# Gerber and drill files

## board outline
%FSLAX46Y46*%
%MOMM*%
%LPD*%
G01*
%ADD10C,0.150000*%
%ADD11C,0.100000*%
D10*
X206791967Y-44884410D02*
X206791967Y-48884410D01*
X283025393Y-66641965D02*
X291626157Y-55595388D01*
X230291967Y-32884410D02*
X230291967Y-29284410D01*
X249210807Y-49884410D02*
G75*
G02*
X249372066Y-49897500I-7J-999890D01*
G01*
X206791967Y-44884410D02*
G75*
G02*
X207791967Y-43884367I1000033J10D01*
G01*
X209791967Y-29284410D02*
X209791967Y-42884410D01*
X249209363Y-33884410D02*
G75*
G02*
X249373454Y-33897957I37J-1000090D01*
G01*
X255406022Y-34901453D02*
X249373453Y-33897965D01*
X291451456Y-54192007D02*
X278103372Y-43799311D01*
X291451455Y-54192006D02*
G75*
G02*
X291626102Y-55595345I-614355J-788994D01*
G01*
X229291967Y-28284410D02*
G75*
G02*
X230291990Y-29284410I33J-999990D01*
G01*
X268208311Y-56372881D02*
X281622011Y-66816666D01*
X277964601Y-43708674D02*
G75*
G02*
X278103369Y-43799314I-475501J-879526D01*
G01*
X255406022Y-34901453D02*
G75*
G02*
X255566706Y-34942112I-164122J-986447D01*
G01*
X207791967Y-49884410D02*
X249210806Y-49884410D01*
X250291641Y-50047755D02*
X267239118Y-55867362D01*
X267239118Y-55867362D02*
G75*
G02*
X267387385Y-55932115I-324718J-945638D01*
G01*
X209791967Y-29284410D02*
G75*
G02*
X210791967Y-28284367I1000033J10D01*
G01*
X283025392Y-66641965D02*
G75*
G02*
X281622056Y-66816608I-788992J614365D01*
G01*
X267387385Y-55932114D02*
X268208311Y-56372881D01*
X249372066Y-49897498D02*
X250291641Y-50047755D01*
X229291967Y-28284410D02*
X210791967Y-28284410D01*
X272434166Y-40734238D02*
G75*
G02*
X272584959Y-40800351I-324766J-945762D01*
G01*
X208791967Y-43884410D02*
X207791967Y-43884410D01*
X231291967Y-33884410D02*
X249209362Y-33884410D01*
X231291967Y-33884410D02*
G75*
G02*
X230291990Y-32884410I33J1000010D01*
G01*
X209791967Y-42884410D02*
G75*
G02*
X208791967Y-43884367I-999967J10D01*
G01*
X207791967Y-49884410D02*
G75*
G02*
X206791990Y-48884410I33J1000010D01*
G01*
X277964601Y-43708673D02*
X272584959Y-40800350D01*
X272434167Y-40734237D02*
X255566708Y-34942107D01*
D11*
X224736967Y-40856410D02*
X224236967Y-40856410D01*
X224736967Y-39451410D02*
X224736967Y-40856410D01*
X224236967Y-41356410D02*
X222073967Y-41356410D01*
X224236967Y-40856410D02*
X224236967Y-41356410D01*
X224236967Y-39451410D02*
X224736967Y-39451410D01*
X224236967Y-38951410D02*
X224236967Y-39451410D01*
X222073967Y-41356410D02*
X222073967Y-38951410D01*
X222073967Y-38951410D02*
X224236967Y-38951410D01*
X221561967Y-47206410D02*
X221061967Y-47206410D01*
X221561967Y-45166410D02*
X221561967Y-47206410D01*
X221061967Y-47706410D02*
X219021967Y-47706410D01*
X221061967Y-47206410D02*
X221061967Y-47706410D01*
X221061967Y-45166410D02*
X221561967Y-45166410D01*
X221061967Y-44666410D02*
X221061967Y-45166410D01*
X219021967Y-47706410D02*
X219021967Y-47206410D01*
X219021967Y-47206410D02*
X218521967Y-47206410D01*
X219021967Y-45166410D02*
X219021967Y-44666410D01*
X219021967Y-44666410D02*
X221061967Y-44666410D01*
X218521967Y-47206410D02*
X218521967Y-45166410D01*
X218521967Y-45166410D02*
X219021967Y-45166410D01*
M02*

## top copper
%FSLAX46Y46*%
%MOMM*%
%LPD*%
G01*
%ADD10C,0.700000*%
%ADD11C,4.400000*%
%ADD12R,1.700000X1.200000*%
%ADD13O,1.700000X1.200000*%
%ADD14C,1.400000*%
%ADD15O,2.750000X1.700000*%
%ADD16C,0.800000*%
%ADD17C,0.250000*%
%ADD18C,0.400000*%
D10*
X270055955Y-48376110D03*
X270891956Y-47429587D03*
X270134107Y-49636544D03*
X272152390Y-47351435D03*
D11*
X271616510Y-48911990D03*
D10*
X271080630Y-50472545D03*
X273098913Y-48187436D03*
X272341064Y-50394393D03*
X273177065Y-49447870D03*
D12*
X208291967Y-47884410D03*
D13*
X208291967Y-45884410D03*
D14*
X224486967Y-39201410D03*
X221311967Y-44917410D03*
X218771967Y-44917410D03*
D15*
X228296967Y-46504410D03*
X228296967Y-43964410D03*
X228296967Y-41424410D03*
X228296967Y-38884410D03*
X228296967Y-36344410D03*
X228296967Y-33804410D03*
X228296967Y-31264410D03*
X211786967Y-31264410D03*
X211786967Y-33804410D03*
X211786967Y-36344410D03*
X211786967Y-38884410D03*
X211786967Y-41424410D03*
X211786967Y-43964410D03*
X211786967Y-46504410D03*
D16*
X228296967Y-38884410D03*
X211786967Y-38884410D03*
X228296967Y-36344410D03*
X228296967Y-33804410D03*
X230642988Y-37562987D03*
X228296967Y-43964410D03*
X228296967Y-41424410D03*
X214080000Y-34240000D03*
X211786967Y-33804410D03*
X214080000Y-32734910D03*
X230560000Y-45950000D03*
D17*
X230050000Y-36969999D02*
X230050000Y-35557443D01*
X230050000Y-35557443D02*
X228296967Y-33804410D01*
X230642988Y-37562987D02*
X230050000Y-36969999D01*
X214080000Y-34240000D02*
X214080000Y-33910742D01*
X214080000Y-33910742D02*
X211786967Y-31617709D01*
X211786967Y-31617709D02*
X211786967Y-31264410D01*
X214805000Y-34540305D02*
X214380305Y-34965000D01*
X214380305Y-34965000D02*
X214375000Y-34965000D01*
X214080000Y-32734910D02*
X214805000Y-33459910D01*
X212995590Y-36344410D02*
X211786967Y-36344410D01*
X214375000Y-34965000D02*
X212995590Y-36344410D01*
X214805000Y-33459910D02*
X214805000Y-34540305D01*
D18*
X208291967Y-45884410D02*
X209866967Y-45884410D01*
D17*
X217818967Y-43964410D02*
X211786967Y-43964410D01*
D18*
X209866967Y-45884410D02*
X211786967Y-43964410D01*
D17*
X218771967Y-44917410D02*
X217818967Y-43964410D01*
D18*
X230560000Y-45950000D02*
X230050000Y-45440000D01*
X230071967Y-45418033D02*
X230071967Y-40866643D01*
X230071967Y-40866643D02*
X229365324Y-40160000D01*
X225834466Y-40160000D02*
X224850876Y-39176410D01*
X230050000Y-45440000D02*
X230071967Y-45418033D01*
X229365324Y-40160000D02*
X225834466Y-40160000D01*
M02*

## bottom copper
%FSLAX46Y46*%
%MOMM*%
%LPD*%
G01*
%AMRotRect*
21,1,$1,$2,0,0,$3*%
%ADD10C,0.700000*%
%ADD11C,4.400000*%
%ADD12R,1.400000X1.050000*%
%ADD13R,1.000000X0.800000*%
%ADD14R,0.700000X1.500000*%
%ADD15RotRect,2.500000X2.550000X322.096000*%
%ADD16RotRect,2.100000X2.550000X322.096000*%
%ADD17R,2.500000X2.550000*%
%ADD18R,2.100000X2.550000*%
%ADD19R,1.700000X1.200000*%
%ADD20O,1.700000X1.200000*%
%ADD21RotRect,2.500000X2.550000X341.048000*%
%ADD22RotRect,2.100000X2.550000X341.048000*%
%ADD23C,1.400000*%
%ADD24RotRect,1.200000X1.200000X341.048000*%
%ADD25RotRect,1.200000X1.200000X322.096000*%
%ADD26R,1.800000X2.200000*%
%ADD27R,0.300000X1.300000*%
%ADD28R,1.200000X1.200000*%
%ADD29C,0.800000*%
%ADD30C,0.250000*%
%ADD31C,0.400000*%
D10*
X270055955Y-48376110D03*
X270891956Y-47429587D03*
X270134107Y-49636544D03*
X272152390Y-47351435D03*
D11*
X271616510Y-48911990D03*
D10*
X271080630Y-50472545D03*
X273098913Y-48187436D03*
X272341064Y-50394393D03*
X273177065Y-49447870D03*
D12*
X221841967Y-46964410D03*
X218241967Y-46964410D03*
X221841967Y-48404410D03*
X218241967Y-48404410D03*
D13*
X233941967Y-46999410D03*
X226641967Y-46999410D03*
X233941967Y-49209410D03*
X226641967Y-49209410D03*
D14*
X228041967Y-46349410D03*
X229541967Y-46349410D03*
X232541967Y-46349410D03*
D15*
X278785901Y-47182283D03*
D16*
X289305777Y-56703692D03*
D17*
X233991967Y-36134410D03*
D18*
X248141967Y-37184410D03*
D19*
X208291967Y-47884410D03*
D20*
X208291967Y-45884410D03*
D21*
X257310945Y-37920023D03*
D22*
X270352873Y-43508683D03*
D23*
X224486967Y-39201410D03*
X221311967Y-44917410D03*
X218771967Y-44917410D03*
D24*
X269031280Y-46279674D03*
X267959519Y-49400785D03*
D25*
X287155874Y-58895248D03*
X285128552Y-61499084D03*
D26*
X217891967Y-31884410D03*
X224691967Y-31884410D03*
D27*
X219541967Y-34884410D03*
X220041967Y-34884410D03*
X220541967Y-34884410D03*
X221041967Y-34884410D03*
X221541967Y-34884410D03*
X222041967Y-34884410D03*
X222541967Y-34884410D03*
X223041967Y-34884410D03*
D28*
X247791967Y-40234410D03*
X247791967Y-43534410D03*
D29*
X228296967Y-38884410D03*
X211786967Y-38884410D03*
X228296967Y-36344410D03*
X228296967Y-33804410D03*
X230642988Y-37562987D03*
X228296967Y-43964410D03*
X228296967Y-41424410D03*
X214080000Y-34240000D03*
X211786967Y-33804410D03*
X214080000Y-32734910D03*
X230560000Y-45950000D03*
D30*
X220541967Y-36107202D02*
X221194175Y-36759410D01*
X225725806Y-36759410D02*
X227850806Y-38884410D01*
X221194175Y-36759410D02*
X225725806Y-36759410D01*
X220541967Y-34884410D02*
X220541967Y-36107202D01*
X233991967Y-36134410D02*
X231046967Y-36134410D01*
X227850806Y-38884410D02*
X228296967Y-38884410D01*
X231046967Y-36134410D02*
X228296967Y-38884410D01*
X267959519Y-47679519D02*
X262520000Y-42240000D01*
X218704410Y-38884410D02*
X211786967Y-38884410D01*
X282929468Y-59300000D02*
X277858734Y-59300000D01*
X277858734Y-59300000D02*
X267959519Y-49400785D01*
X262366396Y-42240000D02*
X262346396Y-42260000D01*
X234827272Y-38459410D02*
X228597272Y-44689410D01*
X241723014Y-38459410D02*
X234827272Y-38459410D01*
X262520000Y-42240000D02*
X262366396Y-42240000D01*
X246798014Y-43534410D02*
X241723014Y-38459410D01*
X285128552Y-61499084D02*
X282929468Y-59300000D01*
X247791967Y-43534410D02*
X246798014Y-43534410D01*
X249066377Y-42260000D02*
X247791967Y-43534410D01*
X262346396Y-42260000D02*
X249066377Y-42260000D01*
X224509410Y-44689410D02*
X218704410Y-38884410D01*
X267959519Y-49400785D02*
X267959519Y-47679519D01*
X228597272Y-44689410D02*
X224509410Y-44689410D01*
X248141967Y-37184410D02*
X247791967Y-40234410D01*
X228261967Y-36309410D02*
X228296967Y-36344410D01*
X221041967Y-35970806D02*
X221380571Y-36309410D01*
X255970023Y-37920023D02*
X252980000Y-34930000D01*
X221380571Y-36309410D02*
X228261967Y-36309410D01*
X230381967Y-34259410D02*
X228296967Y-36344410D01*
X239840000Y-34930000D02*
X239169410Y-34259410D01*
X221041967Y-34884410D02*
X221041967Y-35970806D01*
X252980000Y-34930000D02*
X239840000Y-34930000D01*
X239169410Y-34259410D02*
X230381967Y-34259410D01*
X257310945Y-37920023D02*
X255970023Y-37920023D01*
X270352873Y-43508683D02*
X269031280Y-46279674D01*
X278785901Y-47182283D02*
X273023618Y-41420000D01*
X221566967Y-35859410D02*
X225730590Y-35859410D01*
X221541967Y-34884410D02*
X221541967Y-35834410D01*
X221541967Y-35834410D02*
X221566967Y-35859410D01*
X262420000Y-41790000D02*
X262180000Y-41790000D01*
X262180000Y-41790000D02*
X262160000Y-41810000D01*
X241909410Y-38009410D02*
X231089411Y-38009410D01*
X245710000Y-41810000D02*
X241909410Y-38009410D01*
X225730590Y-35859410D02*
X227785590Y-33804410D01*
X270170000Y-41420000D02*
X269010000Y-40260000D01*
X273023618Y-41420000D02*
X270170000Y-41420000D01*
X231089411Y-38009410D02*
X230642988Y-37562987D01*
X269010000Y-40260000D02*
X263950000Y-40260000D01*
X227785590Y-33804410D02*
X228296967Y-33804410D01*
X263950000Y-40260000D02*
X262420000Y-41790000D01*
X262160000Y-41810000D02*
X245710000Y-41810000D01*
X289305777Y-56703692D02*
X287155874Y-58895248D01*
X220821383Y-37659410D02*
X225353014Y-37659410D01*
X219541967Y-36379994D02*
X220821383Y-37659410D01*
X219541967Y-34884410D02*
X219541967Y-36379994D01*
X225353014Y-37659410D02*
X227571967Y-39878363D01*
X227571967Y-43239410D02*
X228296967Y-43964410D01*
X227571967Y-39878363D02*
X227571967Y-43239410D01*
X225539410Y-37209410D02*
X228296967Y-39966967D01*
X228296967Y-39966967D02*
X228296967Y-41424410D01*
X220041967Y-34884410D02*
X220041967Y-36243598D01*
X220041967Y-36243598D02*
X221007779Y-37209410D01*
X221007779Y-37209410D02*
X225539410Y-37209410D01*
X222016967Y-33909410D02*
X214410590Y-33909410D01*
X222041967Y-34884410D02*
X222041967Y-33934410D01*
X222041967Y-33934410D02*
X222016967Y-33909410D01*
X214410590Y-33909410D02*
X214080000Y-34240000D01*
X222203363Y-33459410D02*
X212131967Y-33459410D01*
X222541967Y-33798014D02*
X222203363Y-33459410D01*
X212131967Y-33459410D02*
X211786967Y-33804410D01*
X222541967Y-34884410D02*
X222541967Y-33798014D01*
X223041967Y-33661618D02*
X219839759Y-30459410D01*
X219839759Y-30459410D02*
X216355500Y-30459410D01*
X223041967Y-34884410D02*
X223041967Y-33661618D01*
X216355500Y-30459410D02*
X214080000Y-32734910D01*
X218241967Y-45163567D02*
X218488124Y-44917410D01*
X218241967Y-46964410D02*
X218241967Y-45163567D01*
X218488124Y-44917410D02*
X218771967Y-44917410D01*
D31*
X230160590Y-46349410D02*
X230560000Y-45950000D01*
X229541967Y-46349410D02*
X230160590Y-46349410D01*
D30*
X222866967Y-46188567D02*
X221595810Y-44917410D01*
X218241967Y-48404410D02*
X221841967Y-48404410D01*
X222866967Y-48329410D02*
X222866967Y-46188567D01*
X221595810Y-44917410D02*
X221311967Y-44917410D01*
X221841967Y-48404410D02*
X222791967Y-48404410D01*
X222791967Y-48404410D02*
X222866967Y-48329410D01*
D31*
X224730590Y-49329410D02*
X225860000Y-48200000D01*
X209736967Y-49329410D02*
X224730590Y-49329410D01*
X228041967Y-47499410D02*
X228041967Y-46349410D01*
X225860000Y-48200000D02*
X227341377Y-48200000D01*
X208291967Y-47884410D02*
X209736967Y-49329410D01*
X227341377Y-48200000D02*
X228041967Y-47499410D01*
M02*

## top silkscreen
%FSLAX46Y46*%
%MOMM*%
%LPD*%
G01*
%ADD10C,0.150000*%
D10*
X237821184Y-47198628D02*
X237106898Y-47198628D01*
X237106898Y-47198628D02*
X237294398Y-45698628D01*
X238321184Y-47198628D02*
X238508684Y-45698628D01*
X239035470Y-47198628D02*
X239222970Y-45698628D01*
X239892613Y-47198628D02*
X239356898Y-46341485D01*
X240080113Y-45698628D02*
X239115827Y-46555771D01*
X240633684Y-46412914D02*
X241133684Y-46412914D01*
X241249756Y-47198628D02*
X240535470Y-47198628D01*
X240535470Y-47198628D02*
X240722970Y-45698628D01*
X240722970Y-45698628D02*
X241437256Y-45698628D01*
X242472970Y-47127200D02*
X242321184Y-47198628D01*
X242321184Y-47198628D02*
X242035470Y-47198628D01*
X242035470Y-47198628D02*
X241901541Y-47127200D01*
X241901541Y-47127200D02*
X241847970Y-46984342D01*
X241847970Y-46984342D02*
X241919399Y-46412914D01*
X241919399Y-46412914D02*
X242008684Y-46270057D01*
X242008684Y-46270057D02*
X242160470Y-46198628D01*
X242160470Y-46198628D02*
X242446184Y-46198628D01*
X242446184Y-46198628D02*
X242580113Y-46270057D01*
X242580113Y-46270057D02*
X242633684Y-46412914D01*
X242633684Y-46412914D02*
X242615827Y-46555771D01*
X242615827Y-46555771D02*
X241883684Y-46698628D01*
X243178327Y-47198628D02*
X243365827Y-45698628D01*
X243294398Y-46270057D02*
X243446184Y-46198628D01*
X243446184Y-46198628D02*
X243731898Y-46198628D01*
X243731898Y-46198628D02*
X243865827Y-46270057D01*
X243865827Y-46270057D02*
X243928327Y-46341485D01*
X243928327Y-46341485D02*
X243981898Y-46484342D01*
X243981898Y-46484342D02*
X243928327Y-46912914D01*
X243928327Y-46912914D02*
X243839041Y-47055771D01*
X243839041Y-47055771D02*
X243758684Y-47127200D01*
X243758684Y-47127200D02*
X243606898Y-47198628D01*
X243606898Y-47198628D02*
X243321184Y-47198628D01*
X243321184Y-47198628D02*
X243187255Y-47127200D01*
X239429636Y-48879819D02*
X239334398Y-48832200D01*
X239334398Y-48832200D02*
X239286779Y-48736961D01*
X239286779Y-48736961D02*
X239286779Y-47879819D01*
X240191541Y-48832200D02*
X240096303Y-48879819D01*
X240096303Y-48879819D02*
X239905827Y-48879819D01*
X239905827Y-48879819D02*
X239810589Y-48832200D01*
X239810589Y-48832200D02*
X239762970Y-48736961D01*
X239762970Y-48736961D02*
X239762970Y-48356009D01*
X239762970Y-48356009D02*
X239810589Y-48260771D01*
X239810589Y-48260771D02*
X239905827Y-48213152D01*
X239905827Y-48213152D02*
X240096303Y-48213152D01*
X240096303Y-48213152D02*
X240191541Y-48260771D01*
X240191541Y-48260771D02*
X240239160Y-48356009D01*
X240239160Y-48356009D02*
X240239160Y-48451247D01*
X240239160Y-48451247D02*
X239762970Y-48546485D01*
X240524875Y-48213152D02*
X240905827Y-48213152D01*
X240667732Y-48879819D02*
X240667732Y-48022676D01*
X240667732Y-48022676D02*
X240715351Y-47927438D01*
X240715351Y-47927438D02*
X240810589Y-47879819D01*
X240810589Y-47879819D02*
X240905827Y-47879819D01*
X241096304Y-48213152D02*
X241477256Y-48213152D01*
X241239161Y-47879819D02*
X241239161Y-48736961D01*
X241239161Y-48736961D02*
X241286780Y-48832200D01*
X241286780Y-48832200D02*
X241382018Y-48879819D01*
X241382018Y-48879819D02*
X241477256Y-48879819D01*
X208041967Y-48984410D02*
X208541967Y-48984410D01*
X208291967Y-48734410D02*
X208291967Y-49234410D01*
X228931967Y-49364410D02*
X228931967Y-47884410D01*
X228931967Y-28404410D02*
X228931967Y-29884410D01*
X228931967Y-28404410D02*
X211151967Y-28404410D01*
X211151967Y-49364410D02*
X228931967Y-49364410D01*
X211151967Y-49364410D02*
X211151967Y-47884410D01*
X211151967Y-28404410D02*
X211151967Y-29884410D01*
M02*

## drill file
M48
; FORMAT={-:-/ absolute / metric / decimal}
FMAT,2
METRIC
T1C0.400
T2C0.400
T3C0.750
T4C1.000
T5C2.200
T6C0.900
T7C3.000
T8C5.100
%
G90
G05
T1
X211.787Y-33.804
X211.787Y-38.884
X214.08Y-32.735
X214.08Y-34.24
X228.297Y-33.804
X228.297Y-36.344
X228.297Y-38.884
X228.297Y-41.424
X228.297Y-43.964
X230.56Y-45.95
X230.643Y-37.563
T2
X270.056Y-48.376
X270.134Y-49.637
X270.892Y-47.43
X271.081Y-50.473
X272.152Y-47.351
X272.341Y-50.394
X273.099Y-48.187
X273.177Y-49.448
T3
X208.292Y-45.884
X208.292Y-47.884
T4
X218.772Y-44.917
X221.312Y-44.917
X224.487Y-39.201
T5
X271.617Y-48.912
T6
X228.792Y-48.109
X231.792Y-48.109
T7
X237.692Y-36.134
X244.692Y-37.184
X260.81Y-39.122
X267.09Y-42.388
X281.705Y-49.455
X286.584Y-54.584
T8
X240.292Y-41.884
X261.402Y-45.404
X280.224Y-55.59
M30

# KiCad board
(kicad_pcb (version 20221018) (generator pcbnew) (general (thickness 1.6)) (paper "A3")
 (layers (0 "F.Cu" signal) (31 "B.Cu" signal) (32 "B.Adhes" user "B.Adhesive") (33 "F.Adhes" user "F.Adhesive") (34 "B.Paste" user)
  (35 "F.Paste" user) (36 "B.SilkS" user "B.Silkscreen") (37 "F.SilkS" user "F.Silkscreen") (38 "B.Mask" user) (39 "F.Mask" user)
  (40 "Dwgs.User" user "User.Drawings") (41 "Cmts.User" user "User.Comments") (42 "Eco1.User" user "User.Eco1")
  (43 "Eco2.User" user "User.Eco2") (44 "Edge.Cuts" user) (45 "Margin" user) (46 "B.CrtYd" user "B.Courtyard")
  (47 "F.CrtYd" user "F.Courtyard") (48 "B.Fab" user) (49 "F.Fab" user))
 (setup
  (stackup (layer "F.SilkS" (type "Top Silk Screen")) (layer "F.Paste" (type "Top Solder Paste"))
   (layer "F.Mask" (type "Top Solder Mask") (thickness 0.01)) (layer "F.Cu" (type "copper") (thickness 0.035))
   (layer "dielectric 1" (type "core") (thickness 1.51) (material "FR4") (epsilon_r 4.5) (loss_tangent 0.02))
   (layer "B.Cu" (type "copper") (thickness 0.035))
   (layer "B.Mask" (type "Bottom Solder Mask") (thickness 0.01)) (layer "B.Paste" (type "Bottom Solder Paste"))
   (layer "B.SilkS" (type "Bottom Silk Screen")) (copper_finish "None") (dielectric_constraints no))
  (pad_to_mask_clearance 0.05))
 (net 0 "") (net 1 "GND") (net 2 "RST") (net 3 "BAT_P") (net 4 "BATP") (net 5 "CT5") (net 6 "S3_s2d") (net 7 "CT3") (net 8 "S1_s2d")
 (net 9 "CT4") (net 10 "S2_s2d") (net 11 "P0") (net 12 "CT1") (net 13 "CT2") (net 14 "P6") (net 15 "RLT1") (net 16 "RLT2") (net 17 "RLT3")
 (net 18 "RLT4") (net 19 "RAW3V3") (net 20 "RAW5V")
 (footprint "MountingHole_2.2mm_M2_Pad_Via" (layer "F.Cu") (at 271.61651 48.91199 -18.952)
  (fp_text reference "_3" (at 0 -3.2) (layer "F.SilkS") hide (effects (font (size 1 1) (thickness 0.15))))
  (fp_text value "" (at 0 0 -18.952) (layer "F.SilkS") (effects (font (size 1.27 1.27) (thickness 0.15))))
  (pad "1" thru_hole circle (at -1.65 0) (size 0.7 0.7) (drill 0.4) (layers "*.Cu" "*.Mask"))
  (pad "1" thru_hole circle (at -1.166726 -1.166726) (size 0.7 0.7) (drill 0.4) (layers "*.Cu" "*.Mask"))
  (pad "1" thru_hole circle (at -1.166726 1.166726) (size 0.7 0.7) (drill 0.4) (layers "*.Cu" "*.Mask"))
  (pad "1" thru_hole circle (at 0 -1.65) (size 0.7 0.7) (drill 0.4) (layers "*.Cu" "*.Mask"))
  (pad "1" thru_hole circle (at 0 0) (size 4.4 4.4) (drill 2.2) (layers "*.Cu" "*.Mask"))
  (pad "1" thru_hole circle (at 0 1.65) (size 0.7 0.7) (drill 0.4) (layers "*.Cu" "*.Mask"))
  (pad "1" thru_hole circle (at 1.166726 -1.166726) (size 0.7 0.7) (drill 0.4) (layers "*.Cu" "*.Mask"))
  (pad "1" thru_hole circle (at 1.166726 1.166726) (size 0.7 0.7) (drill 0.4) (layers "*.Cu" "*.Mask"))
  (pad "1" thru_hole circle (at 1.65 0) (size 0.7 0.7) (drill 0.4) (layers "*.Cu" "*.Mask")))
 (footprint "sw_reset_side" (layer "F.Cu") (at 220.041967 47.68441 -90)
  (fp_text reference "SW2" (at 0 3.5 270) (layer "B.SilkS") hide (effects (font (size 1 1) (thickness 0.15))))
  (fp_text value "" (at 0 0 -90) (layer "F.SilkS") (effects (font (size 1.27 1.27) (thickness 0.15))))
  (pad "1" smd rect (at -0.72 -1.8 180) (size 1.4 1.05) (layers "B.Cu" "B.Paste" "B.Mask") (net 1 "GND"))
  (pad "1" smd rect (at -0.72 1.8 180) (size 1.4 1.05) (layers "B.Cu" "B.Paste" "B.Mask") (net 1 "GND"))
  (pad "2" smd rect (at 0.72 -1.8 180) (size 1.4 1.05) (layers "B.Cu" "B.Paste" "B.Mask") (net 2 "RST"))
  (pad "2" smd rect (at 0.72 1.8 180) (size 1.4 1.05) (layers "B.Cu" "B.Paste" "B.Mask") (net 2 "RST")))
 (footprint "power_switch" (layer "F.Cu") (at 230.291967 48.08441 -90)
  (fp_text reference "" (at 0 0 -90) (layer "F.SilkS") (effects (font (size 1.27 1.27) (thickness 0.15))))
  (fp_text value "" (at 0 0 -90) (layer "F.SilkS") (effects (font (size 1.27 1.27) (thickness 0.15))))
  (pad "" smd rect (at -1.085 -3.65 180) (size 1 0.8) (layers "B.Cu" "B.Paste" "B.Mask"))
  (pad "" smd rect (at -1.085 3.65 180) (size 1 0.8) (layers "B.Cu" "B.Paste" "B.Mask"))
  (pad "" np_thru_hole circle (at 0.025 -1.5) (size 0.9 0.9) (drill 0.9) (layers "*.Cu" "*.Mask"))
  (pad "" np_thru_hole circle (at 0.025 1.5) (size 0.9 0.9) (drill 0.9) (layers "*.Cu" "*.Mask"))
  (pad "" smd rect (at 1.125 -3.65 180) (size 1 0.8) (layers "B.Cu" "B.Paste" "B.Mask"))
  (pad "" smd rect (at 1.125 3.65 180) (size 1 0.8) (layers "B.Cu" "B.Paste" "B.Mask"))
  (pad "4" smd rect (at -1.735 2.25 180) (size 0.7 1.5) (layers "B.Cu" "B.Paste" "B.Mask") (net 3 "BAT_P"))
  (pad "5" smd rect (at -1.735 0.75 180) (size 0.7 1.5) (layers "B.Cu" "B.Paste" "B.Mask") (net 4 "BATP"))
  (pad "6" smd rect (at -1.735 -2.25 180) (size 0.7 1.5) (layers "B.Cu" "B.Paste" "B.Mask")))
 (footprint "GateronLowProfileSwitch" (layer "F.Cu") (at 280.224404 55.589614 -37.904)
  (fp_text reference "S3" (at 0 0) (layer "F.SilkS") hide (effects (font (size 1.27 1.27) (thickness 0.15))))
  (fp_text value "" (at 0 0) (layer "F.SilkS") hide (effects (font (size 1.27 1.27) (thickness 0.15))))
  (pad "" np_thru_hole circle (at -2.6 -5.75) (size 3 3) (drill 3) (layers "*.Cu" "*.Mask"))
  (pad "" np_thru_hole circle (at 0 0) (size 5.1 5.1) (drill 5.1) (layers "*.Cu" "*.Mask"))
  (pad "" np_thru_hole circle (at 4.4 -4.7) (size 3 3) (drill 3) (layers "*.Cu" "*.Mask"))
  (pad "1" smd rect (at -6.3 -5.75 322.096) (size 2.5 2.55) (layers "B.Cu" "B.Paste" "B.Mask") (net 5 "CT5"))
  (pad "2" smd rect (at 7.85 -4.7 322.096) (size 2.1 2.55) (layers "B.Cu" "B.Paste" "B.Mask") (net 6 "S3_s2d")))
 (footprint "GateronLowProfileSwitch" (layer "F.Cu") (at 240.291967 41.88441)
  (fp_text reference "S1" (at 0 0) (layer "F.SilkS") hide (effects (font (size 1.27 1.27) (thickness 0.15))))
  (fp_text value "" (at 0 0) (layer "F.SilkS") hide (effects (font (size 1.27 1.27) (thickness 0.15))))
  (pad "" np_thru_hole circle (at -2.6 -5.75) (size 3 3) (drill 3) (layers "*.Cu" "*.Mask"))
  (pad "" np_thru_hole circle (at 0 0) (size 5.1 5.1) (drill 5.1) (layers "*.Cu" "*.Mask"))
  (pad "" np_thru_hole circle (at 4.4 -4.7) (size 3 3) (drill 3) (layers "*.Cu" "*.Mask"))
  (pad "1" smd rect (at -6.3 -5.75) (size 2.5 2.55) (layers "B.Cu" "B.Paste" "B.Mask") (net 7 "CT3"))
  (pad "2" smd rect (at 7.85 -4.7) (size 2.1 2.55) (layers "B.Cu" "B.Paste" "B.Mask") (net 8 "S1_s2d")))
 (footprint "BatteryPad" (layer "F.Cu") (at 208.291967 46.88441 90)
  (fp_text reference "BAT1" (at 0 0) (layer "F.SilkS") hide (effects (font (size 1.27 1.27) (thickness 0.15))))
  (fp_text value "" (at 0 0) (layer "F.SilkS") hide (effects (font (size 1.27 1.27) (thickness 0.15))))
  (fp_line (start -2.1 -0.25) (end -2.1 0.25) (stroke (width 0.15) (type solid)) (layer "F.SilkS"))
  (fp_line (start -1.85 0) (end -2.35 0) (stroke (width 0.15) (type solid)) (layer "F.SilkS"))
  (pad "1" thru_hole rect (at -1 0 90) (size 1.2 1.7) (drill 0.75) (layers "*.Cu" "*.Mask") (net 3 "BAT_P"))
  (pad "2" thru_hole oval (at 1 0 90) (size 1.2 1.7) (drill 0.75) (layers "*.Cu" "*.Mask") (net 1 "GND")))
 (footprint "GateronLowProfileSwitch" (layer "F.Cu") (at 261.401967 45.40441 -18.952)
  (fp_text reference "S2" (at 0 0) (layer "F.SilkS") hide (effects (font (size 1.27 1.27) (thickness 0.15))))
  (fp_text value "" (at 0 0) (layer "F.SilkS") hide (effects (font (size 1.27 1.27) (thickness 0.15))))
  (pad "" np_thru_hole circle (at -2.6 -5.75) (size 3 3) (drill 3) (layers "*.Cu" "*.Mask"))
  (pad "" np_thru_hole circle (at 0 0) (size 5.1 5.1) (drill 5.1) (layers "*.Cu" "*.Mask"))
  (pad "" np_thru_hole circle (at 4.4 -4.7) (size 3 3) (drill 3) (layers "*.Cu" "*.Mask"))
  (pad "1" smd rect (at -6.3 -5.75 341.048) (size 2.5 2.55) (layers "B.Cu" "B.Paste" "B.Mask") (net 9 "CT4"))
  (pad "2" smd rect (at 7.85 -4.7 341.048) (size 2.1 2.55) (layers "B.Cu" "B.Paste" "B.Mask") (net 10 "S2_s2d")))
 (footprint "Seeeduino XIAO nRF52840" (layer "F.Cu") (at 220.041967 38.88441 180)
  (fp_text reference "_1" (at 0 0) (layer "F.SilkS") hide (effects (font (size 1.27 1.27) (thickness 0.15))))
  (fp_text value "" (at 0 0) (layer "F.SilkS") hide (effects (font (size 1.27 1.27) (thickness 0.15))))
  (fp_line (start -8.89 -10.48) (end -8.89 -9) (stroke (width 0.15) (type solid)) (layer "F.SilkS"))
  (fp_line (start -8.89 10.48) (end -8.89 9) (stroke (width 0.15) (type solid)) (layer "F.SilkS"))
  (fp_line (start -8.89 10.48) (end 8.89 10.48) (stroke (width 0.15) (type solid)) (layer "F.SilkS"))
  (fp_line (start 8.89 -10.48) (end -8.89 -10.48) (stroke (width 0.15) (type solid)) (layer "F.SilkS"))
  (fp_line (start 8.89 -10.48) (end 8.89 -9) (stroke (width 0.15) (type solid)) (layer "F.SilkS"))
  (fp_line (start 8.89 10.48) (end 8.89 9) (stroke (width 0.15) (type solid)) (layer "F.SilkS"))
  (fp_line (start -4.695 -1.972) (end -4.195 -1.972) (stroke (width 0.1) (type solid)) (layer "Edge.Cuts"))
  (fp_line (start -4.695 -0.567) (end -4.695 -1.972) (stroke (width 0.1) (type solid)) (layer "Edge.Cuts"))
  (fp_line (start -4.195 -2.472) (end -2.032 -2.472) (stroke (width 0.1) (type solid)) (layer "Edge.Cuts"))
  (fp_line (start -4.195 -1.972) (end -4.195 -2.472) (stroke (width 0.1) (type solid)) (layer "Edge.Cuts"))
  (fp_line (start -4.195 -0.567) (end -4.695 -0.567) (stroke (width 0.1) (type solid)) (layer "Edge.Cuts"))
  (fp_line (start -4.195 -0.067) (end -4.195 -0.567) (stroke (width 0.1) (type solid)) (layer "Edge.Cuts"))
  (fp_line (start -2.032 -2.472) (end -2.032 -0.067) (stroke (width 0.1) (type solid)) (layer "Edge.Cuts"))
  (fp_line (start -2.032 -0.067) (end -4.195 -0.067) (stroke (width 0.1) (type solid)) (layer "Edge.Cuts"))
  (fp_line (start -1.52 -8.322) (end -1.02 -8.322) (stroke (width 0.1) (type solid)) (layer "Edge.Cuts"))
  (fp_line (start -1.52 -6.282) (end -1.52 -8.322) (stroke (width 0.1) (type solid)) (layer "Edge.Cuts"))
  (fp_line (start -1.02 -8.822) (end 1.02 -8.822) (stroke (width 0.1) (type solid)) (layer "Edge.Cuts"))
  (fp_line (start -1.02 -8.322) (end -1.02 -8.822) (stroke (width 0.1) (type solid)) (layer "Edge.Cuts"))
  (fp_line (start -1.02 -6.282) (end -1.52 -6.282) (stroke (width 0.1) (type solid)) (layer "Edge.Cuts"))
  (fp_line (start -1.02 -5.782) (end -1.02 -6.282) (stroke (width 0.1) (type solid)) (layer "Edge.Cuts"))
  (fp_line (start 1.02 -8.822) (end 1.02 -8.322) (stroke (width 0.1) (type solid)) (layer "Edge.Cuts"))
  (fp_line (start 1.02 -8.322) (end 1.52 -8.322) (stroke (width 0.1) (type solid)) (layer "Edge.Cuts"))
  (fp_line (start 1.02 -6.282) (end 1.02 -5.782) (stroke (width 0.1) (type solid)) (layer "Edge.Cuts"))
  (fp_line (start 1.02 -5.782) (end -1.02 -5.782) (stroke (width 0.1) (type solid)) (layer "Edge.Cuts"))
  (fp_line (start 1.52 -8.322) (end 1.52 -6.282) (stroke (width 0.1) (type solid)) (layer "Edge.Cuts"))
  (fp_line (start 1.52 -6.282) (end 1.02 -6.282) (stroke (width 0.1) (type solid)) (layer "Edge.Cuts"))
  (pad "" thru_hole circle (at -4.445 -0.317) (size 1.4 1.4) (drill 1) (layers "*.Cu" "*.Mask") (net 4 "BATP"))
  (pad "" thru_hole circle (at -1.27 -6.033) (size 1.4 1.4) (drill 1) (layers "*.Cu" "*.Mask") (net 2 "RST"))
  (pad "" thru_hole circle (at 1.27 -6.033) (size 1.4 1.4) (drill 1) (layers "*.Cu" "*.Mask") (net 1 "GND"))
  (pad "1" smd oval (at -8.255 -7.62 180) (size 2.75 1.7) (layers "F.Cu" "F.Paste" "F.Mask") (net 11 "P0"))
  (pad "2" smd oval (at -8.255 -5.08 180) (size 2.75 1.7) (layers "F.Cu" "F.Paste" "F.Mask") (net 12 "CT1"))
  (pad "3" smd oval (at -8.255 -2.54 180) (size 2.75 1.7) (layers "F.Cu" "F.Paste" "F.Mask") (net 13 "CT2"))
  (pad "4" smd oval (at -8.255 0 180) (size 2.75 1.7) (layers "F.Cu" "F.Paste" "F.Mask") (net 7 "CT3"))
  (pad "5" smd oval (at -8.255 2.54 180) (size 2.75 1.7) (layers "F.Cu" "F.Paste" "F.Mask") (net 9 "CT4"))
  (pad "6" smd oval (at -8.255 5.08 180) (size 2.75 1.7) (layers "F.Cu" "F.Paste" "F.Mask") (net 5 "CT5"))
  (pad "7" smd oval (at -8.255 7.62 180) (size 2.75 1.7) (layers "F.Cu" "F.Paste" "F.Mask") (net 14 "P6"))
  (pad "8" smd oval (at 8.255 7.62 180) (size 2.75 1.7) (layers "F.Cu" "F.Paste" "F.Mask") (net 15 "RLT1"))
  (pad "9" smd oval (at 8.255 5.08 180) (size 2.75 1.7) (layers "F.Cu" "F.Paste" "F.Mask") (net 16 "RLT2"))
  (pad "10" smd oval (at 8.255 2.54 180) (size 2.75 1.7) (layers "F.Cu" "F.Paste" "F.Mask") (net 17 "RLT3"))
  (pad "11" smd oval (at 8.255 0 180) (size 2.75 1.7) (layers "F.Cu" "F.Paste" "F.Mask") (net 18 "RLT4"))
  (pad "12" smd oval (at 8.255 -2.54 180) (size 2.75 1.7) (layers "F.Cu" "F.Paste" "F.Mask") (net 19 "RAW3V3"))
  (pad "13" smd oval (at 8.255 -5.08 180) (size 2.75 1.7) (layers "F.Cu" "F.Paste" "F.Mask") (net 1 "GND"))
  (pad "14" smd oval (at 8.255 -7.62 180) (size 2.75 1.7) (layers "F.Cu" "F.Paste" "F.Mask") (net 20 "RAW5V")))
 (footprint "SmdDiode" (layer "B.Cu") (at 261.401967 45.40441 -18.952)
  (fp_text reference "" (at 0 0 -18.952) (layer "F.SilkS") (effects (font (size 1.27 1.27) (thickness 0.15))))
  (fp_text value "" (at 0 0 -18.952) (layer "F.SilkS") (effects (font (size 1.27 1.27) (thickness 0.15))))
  (pad "1" smd rect (at 7.5 -1.65 341.048) (size 1.2 1.2) (layers "B.Cu" "B.Paste" "B.Mask") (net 10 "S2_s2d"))
  (pad "2" smd rect (at 7.5 1.65 341.048) (size 1.2 1.2) (layers "B.Cu" "B.Paste" "B.Mask") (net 18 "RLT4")))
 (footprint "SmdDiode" (layer "B.Cu") (at 280.224404 55.589614 -37.904)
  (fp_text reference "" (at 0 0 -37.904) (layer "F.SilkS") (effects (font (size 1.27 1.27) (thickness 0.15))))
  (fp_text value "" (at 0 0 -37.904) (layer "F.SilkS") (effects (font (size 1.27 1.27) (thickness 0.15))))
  (pad "1" smd rect (at 7.5 -1.65 322.096) (size 1.2 1.2) (layers "B.Cu" "B.Paste" "B.Mask") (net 6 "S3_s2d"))
  (pad "2" smd rect (at 7.5 1.65 322.096) (size 1.2 1.2) (layers "B.Cu" "B.Paste" "B.Mask") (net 18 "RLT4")))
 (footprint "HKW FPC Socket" (layer "B.Cu") (at 221.291967 31.88441)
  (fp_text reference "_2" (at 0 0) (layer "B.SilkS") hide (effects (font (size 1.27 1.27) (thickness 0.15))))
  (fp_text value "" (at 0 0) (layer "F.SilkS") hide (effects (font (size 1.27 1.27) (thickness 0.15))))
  (pad "" smd rect (at -3.4 0) (size 1.8 2.2) (layers "B.Cu" "B.Paste" "B.Mask"))
  (pad "" smd rect (at 3.4 0) (size 1.8 2.2) (layers "B.Cu" "B.Paste" "B.Mask"))
  (pad "1" smd rect (at -1.75 3) (size 0.3 1.3) (layers "B.Cu" "B.Paste" "B.Mask") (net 12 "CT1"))
  (pad "2" smd rect (at -1.25 3) (size 0.3 1.3) (layers "B.Cu" "B.Paste" "B.Mask") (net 13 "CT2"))
  (pad "3" smd rect (at -0.75 3) (size 0.3 1.3) (layers "B.Cu" "B.Paste" "B.Mask") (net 7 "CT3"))
  (pad "4" smd rect (at -0.25 3) (size 0.3 1.3) (layers "B.Cu" "B.Paste" "B.Mask") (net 9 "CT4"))
  (pad "5" smd rect (at 0.25 3) (size 0.3 1.3) (layers "B.Cu" "B.Paste" "B.Mask") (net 5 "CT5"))
  (pad "6" smd rect (at 0.75 3) (size 0.3 1.3) (layers "B.Cu" "B.Paste" "B.Mask") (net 15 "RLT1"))
  (pad "7" smd rect (at 1.25 3) (size 0.3 1.3) (layers "B.Cu" "B.Paste" "B.Mask") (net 16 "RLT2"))
  (pad "8" smd rect (at 1.75 3) (size 0.3 1.3) (layers "B.Cu" "B.Paste" "B.Mask") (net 17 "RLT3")))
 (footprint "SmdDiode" (layer "B.Cu") (at 240.291967 41.88441)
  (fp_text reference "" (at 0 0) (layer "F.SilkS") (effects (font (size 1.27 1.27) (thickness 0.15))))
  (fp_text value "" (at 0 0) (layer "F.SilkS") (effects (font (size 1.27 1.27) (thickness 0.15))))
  (pad "1" smd rect (at 7.5 -1.65) (size 1.2 1.2) (layers "B.Cu" "B.Paste" "B.Mask") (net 8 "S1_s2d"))
  (pad "2" smd rect (at 7.5 1.65) (size 1.2 1.2) (layers "B.Cu" "B.Paste" "B.Mask") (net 18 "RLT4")))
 (gr_line (start 206.791967 44.88441) (end 206.791967 48.88441) (stroke (width 0.15) (type solid)) (layer "Edge.Cuts"))
 (gr_line (start 283.025393 66.641965) (end 291.626157 55.595388) (stroke (width 0.15) (type solid)) (layer "Edge.Cuts"))
 (gr_line (start 230.291967 32.88441) (end 230.291967 29.28441) (stroke (width 0.15) (type solid)) (layer "Edge.Cuts"))
 (gr_arc (start 249.210807 49.88441) (mid 249.291702 49.887687) (end 249.372066 49.897498) (stroke (width 0.15) (type solid))
  (layer "Edge.Cuts"))
 (gr_arc (start 206.791967 44.88441) (mid 207.08486 44.177303) (end 207.791967 43.88441) (stroke (width 0.15) (type solid))
  (layer "Edge.Cuts"))
 (gr_line (start 209.791967 29.28441) (end 209.791967 42.88441) (stroke (width 0.15) (type solid)) (layer "Edge.Cuts"))
 (gr_arc (start 249.209363 33.88441) (mid 249.291687 33.887805) (end 249.373453 33.897965) (stroke (width 0.15) (type solid))
  (layer "Edge.Cuts"))
 (gr_line (start 255.406022 34.901453) (end 249.373453 33.897965) (stroke (width 0.15) (type solid)) (layer "Edge.Cuts"))
 (gr_line (start 291.451456 54.192007) (end 278.103372 43.799311) (stroke (width 0.15) (type solid)) (layer "Edge.Cuts"))
 (gr_arc (start 291.451455 54.192006) (mid 291.829456 54.857515) (end 291.626157 55.595388) (stroke (width 0.15) (type solid))
  (layer "Edge.Cuts"))
 (gr_arc (start 229.291967 28.28441) (mid 229.999074 28.577303) (end 230.291967 29.28441) (stroke (width 0.15) (type solid))
  (layer "Edge.Cuts"))
 (gr_line (start 268.208311 56.372881) (end 281.622011 66.816666) (stroke (width 0.15) (type solid)) (layer "Edge.Cuts"))
 (gr_arc (start 277.964601 43.708674) (mid 278.035868 43.751112) (end 278.103372 43.799311) (stroke (width 0.15) (type solid))
  (layer "Edge.Cuts"))
 (gr_arc (start 255.406022 34.901453) (mid 255.487209 34.918445) (end 255.566708 34.942107) (stroke (width 0.15) (type solid))
  (layer "Edge.Cuts"))
 (gr_line (start 207.791967 49.88441) (end 249.210806 49.88441) (stroke (width 0.15) (type solid)) (layer "Edge.Cuts"))
 (gr_line (start 250.291641 50.047755) (end 267.239118 55.867362) (stroke (width 0.15) (type solid)) (layer "Edge.Cuts"))
 (gr_arc (start 267.239118 55.867362) (mid 267.314563 55.896734) (end 267.387385 55.932114) (stroke (width 0.15) (type solid))
  (layer "Edge.Cuts"))
 (gr_arc (start 209.791967 29.28441) (mid 210.08486 28.577303) (end 210.791967 28.28441) (stroke (width 0.15) (type solid))
  (layer "Edge.Cuts"))
 (gr_arc (start 283.025392 66.641965) (mid 282.359883 67.019965) (end 281.622011 66.816666) (stroke (width 0.15) (type solid))
  (layer "Edge.Cuts"))
 (gr_line (start 267.387385 55.932114) (end 268.208311 56.372881) (stroke (width 0.15) (type solid)) (layer "Edge.Cuts"))
 (gr_line (start 249.372066 49.897498) (end 250.291641 50.047755) (stroke (width 0.15) (type solid)) (layer "Edge.Cuts"))
 (gr_line (start 229.291967 28.28441) (end 210.791967 28.28441) (stroke (width 0.15) (type solid)) (layer "Edge.Cuts"))
 (gr_arc (start 272.434166 40.734238) (mid 272.510925 40.764185) (end 272.584959 40.80035) (stroke (width 0.15) (type solid))
  (layer "Edge.Cuts"))
 (gr_line (start 208.791967 43.88441) (end 207.791967 43.88441) (stroke (width 0.15) (type solid)) (layer "Edge.Cuts"))
 (gr_line (start 231.291967 33.88441) (end 249.209362 33.88441) (stroke (width 0.15) (type solid)) (layer "Edge.Cuts"))
 (gr_arc (start 231.291967 33.88441) (mid 230.58486 33.591517) (end 230.291967 32.88441) (stroke (width 0.15) (type solid))
  (layer "Edge.Cuts"))
 (gr_arc (start 209.791967 42.88441) (mid 209.499074 43.591517) (end 208.791967 43.88441) (stroke (width 0.15) (type solid))
  (layer "Edge.Cuts"))
 (gr_arc (start 207.791967 49.88441) (mid 207.08486 49.591517) (end 206.791967 48.88441) (stroke (width 0.15) (type solid))
  (layer "Edge.Cuts"))
 (gr_line (start 277.964601 43.708673) (end 272.584959 40.80035) (stroke (width 0.15) (type solid)) (layer "Edge.Cuts"))
 (gr_line (start 272.434167 40.734237) (end 255.566708 34.942107) (stroke (width 0.15) (type solid)) (layer "Edge.Cuts"))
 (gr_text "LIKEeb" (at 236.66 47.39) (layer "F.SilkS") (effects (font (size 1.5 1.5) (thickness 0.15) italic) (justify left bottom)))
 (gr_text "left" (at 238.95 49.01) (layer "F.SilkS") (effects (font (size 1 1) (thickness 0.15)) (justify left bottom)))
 (via (at 228.296967 38.88441) (size 0.8) (drill 0.4) (layers "F.Cu" "B.Cu") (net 7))
 (segment (start 220.541967 36.107202) (end 221.194175 36.75941) (width 0.25) (layer "B.Cu") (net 7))
 (segment (start 225.725806 36.75941) (end 227.850806 38.88441) (width 0.25) (layer "B.Cu") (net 7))
 (segment (start 221.194175 36.75941) (end 225.725806 36.75941) (width 0.25) (layer "B.Cu") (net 7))
 (segment (start 220.541967 34.88441) (end 220.541967 36.107202) (width 0.25) (layer "B.Cu") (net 7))
 (segment (start 233.991967 36.13441) (end 231.046967 36.13441) (width 0.25) (layer "B.Cu") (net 7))
 (segment (start 227.850806 38.88441) (end 228.296967 38.88441) (width 0.25) (layer "B.Cu") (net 7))
 (segment (start 231.046967 36.13441) (end 228.296967 38.88441) (width 0.25) (layer "B.Cu") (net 7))
 (via (at 211.786967 38.88441) (size 0.8) (drill 0.4) (layers "F.Cu" "B.Cu") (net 18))
 (segment (start 267.959519 47.679519) (end 262.52 42.24) (width 0.25) (layer "B.Cu") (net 18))
 (segment (start 218.70441 38.88441) (end 211.786967 38.88441) (width 0.25) (layer "B.Cu") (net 18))
 (segment (start 282.929468 59.3) (end 277.858734 59.3) (width 0.25) (layer "B.Cu") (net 18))
 (segment (start 277.858734 59.3) (end 267.959519 49.400785) (width 0.25) (layer "B.Cu") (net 18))
 (segment (start 262.366396 42.24) (end 262.346396 42.26) (width 0.25) (layer "B.Cu") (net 18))
 (segment (start 234.827272 38.45941) (end 228.597272 44.68941) (width 0.25) (layer "B.Cu") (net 18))
 (segment (start 241.723014 38.45941) (end 234.827272 38.45941) (width 0.25) (layer "B.Cu") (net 18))
 (segment (start 262.52 42.24) (end 262.366396 42.24) (width 0.25) (layer "B.Cu") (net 18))
 (segment (start 246.798014 43.53441) (end 241.723014 38.45941) (width 0.25) (layer "B.Cu") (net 18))
 (segment (start 285.128552 61.499084) (end 282.929468 59.3) (width 0.25) (layer "B.Cu") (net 18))
 (segment (start 247.791967 43.53441) (end 246.798014 43.53441) (width 0.25) (layer "B.Cu") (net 18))
 (segment (start 249.066377 42.26) (end 247.791967 43.53441) (width 0.25) (layer "B.Cu") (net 18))
 (segment (start 262.346396 42.26) (end 249.066377 42.26) (width 0.25) (layer "B.Cu") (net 18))
 (segment (start 224.50941 44.68941) (end 218.70441 38.88441) (width 0.25) (layer "B.Cu") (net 18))
 (segment (start 267.959519 49.400785) (end 267.959519 47.679519) (width 0.25) (layer "B.Cu") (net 18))
 (segment (start 228.597272 44.68941) (end 224.50941 44.68941) (width 0.25) (layer "B.Cu") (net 18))
 (segment (start 248.141967 37.18441) (end 247.791967 40.23441) (width 0.25) (layer "B.Cu") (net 8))
 (via (at 228.296967 36.34441) (size 0.8) (drill 0.4) (layers "F.Cu" "B.Cu") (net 9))
 (segment (start 228.261967 36.30941) (end 228.296967 36.34441) (width 0.25) (layer "B.Cu") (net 9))
 (segment (start 221.041967 35.970806) (end 221.380571 36.30941) (width 0.25) (layer "B.Cu") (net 9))
 (segment (start 255.970023 37.920023) (end 252.98 34.93) (width 0.25) (layer "B.Cu") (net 9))
 (segment (start 221.380571 36.30941) (end 228.261967 36.30941) (width 0.25) (layer "B.Cu") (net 9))
 (segment (start 230.381967 34.25941) (end 228.296967 36.34441) (width 0.25) (layer "B.Cu") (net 9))
 (segment (start 239.84 34.93) (end 239.16941 34.25941) (width 0.25) (layer "B.Cu") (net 9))
 (segment (start 221.041967 34.88441) (end 221.041967 35.970806) (width 0.25) (layer "B.Cu") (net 9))
 (segment (start 252.98 34.93) (end 239.84 34.93) (width 0.25) (layer "B.Cu") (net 9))
 (segment (start 239.16941 34.25941) (end 230.381967 34.25941) (width 0.25) (layer "B.Cu") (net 9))
 (segment (start 257.310945 37.920023) (end 255.970023 37.920023) (width 0.25) (layer "B.Cu") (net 9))
 (segment (start 270.352873 43.508683) (end 269.03128 46.279674) (width 0.25) (layer "B.Cu") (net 10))
 (segment (start 230.05 36.969999) (end 230.05 35.557443) (width 0.25) (layer "F.Cu") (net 5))
 (segment (start 230.05 35.557443) (end 228.296967 33.80441) (width 0.25) (layer "F.Cu") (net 5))
 (segment (start 230.642988 37.562987) (end 230.05 36.969999) (width 0.25) (layer "F.Cu") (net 5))
 (via (at 228.296967 33.80441) (size 0.8) (drill 0.4) (layers "F.Cu" "B.Cu") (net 5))
 (via (at 230.642988 37.562987) (size 0.8) (drill 0.4) (layers "F.Cu" "B.Cu") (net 5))
 (segment (start 278.785901 47.182283) (end 273.023618 41.42) (width 0.25) (layer "B.Cu") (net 5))
 (segment (start 221.566967 35.85941) (end 225.73059 35.85941) (width 0.25) (layer "B.Cu") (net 5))
 (segment (start 221.541967 34.88441) (end 221.541967 35.83441) (width 0.25) (layer "B.Cu") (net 5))
 (segment (start 221.541967 35.83441) (end 221.566967 35.85941) (width 0.25) (layer "B.Cu") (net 5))
 (segment (start 262.42 41.79) (end 262.18 41.79) (width 0.25) (layer "B.Cu") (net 5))
 (segment (start 262.18 41.79) (end 262.16 41.81) (width 0.25) (layer "B.Cu") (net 5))
 (segment (start 241.90941 38.00941) (end 231.089411 38.00941) (width 0.25) (layer "B.Cu") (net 5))
 (segment (start 245.71 41.81) (end 241.90941 38.00941) (width 0.25) (layer "B.Cu") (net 5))
 (segment (start 225.73059 35.85941) (end 227.78559 33.80441) (width 0.25) (layer "B.Cu") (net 5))
 (segment (start 270.17 41.42) (end 269.01 40.26) (width 0.25) (layer "B.Cu") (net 5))
 (segment (start 273.023618 41.42) (end 270.17 41.42) (width 0.25) (layer "B.Cu") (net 5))
 (segment (start 231.089411 38.00941) (end 230.642988 37.562987) (width 0.25) (layer "B.Cu") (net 5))
 (segment (start 269.01 40.26) (end 263.95 40.26) (width 0.25) (layer "B.Cu") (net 5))
 (segment (start 227.78559 33.80441) (end 228.296967 33.80441) (width 0.25) (layer "B.Cu") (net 5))
 (segment (start 263.95 40.26) (end 262.42 41.79) (width 0.25) (layer "B.Cu") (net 5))
 (segment (start 262.16 41.81) (end 245.71 41.81) (width 0.25) (layer "B.Cu") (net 5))
 (segment (start 289.305777 56.703692) (end 287.155874 58.895248) (width 0.25) (layer "B.Cu") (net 6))
 (via (at 228.296967 43.96441) (size 0.8) (drill 0.4) (layers "F.Cu" "B.Cu") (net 12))
 (segment (start 220.821383 37.65941) (end 225.353014 37.65941) (width 0.25) (layer "B.Cu") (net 12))
 (segment (start 219.541967 36.379994) (end 220.821383 37.65941) (width 0.25) (layer "B.Cu") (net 12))
 (segment (start 219.541967 34.88441) (end 219.541967 36.379994) (width 0.25) (layer "B.Cu") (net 12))
 (segment (start 225.353014 37.65941) (end 227.571967 39.878363) (width 0.25) (layer "B.Cu") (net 12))
 (segment (start 227.571967 43.23941) (end 228.296967 43.96441) (width 0.25) (layer "B.Cu") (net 12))
 (segment (start 227.571967 39.878363) (end 227.571967 43.23941) (width 0.25) (layer "B.Cu") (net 12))
 (via (at 228.296967 41.42441) (size 0.8) (drill 0.4) (layers "F.Cu" "B.Cu") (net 13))
 (segment (start 225.53941 37.20941) (end 228.296967 39.966967) (width 0.25) (layer "B.Cu") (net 13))
 (segment (start 228.296967 39.966967) (end 228.296967 41.42441) (width 0.25) (layer "B.Cu") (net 13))
 (segment (start 220.041967 34.88441) (end 220.041967 36.243598) (width 0.25) (layer "B.Cu") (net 13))
 (segment (start 220.041967 36.243598) (end 221.007779 37.20941) (width 0.25) (layer "B.Cu") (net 13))
 (segment (start 221.007779 37.20941) (end 225.53941 37.20941) (width 0.25) (layer "B.Cu") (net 13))
 (segment (start 214.08 34.24) (end 214.08 33.910742) (width 0.25) (layer "F.Cu") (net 15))
 (segment (start 214.08 33.910742) (end 211.786967 31.617709) (width 0.25) (layer "F.Cu") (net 15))
 (segment (start 211.786967 31.617709) (end 211.786967 31.26441) (width 0.25) (layer "F.Cu") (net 15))
 (via (at 214.08 34.24) (size 0.8) (drill 0.4) (layers "F.Cu" "B.Cu") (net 15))
 (segment (start 222.016967 33.90941) (end 214.41059 33.90941) (width 0.25) (layer "B.Cu") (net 15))
 (segment (start 222.041967 34.88441) (end 222.041967 33.93441) (width 0.25) (layer "B.Cu") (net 15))
 (segment (start 222.041967 33.93441) (end 222.016967 33.90941) (width 0.25) (layer "B.Cu") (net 15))
 (segment (start 214.41059 33.90941) (end 214.08 34.24) (width 0.25) (layer "B.Cu") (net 15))
 (via (at 211.786967 33.80441) (size 0.8) (drill 0.4) (layers "F.Cu" "B.Cu") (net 16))
 (segment (start 222.203363 33.45941) (end 212.131967 33.45941) (width 0.25) (layer "B.Cu") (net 16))
 (segment (start 222.541967 33.798014) (end 222.203363 33.45941) (width 0.25) (layer "B.Cu") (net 16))
 (segment (start 212.131967 33.45941) (end 211.786967 33.80441) (width 0.25) (layer "B.Cu") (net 16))
 (segment (start 222.541967 34.88441) (end 222.541967 33.798014) (width 0.25) (layer "B.Cu") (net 16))
 (segment (start 214.805 34.540305) (end 214.380305 34.965) (width 0.25) (layer "F.Cu") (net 17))
 (segment (start 214.380305 34.965) (end 214.375 34.965) (width 0.25) (layer "F.Cu") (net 17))
 (segment (start 214.08 32.73491) (end 214.805 33.45991) (width 0.25) (layer "F.Cu") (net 17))
 (segment (start 212.99559 36.34441) (end 211.786967 36.34441) (width 0.25) (layer "F.Cu") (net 17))
 (segment (start 214.375 34.965) (end 212.99559 36.34441) (width 0.25) (layer "F.Cu") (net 17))
 (segment (start 214.805 33.45991) (end 214.805 34.540305) (width 0.25) (layer "F.Cu") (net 17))
 (via (at 214.08 32.73491) (size 0.8) (drill 0.4) (layers "F.Cu" "B.Cu") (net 17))
 (segment (start 223.041967 33.661618) (end 219.839759 30.45941) (width 0.25) (layer "B.Cu") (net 17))
 (segment (start 219.839759 30.45941) (end 216.3555 30.45941) (width 0.25) (layer "B.Cu") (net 17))
 (segment (start 223.041967 34.88441) (end 223.041967 33.661618) (width 0.25) (layer "B.Cu") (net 17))
 (segment (start 216.3555 30.45941) (end 214.08 32.73491) (width 0.25) (layer "B.Cu") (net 17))
 (segment (start 208.291967 45.88441) (end 209.866967 45.88441) (width 0.4) (layer "F.Cu") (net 1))
 (segment (start 217.818967 43.96441) (end 211.786967 43.96441) (width 0.25) (layer "F.Cu") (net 1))
 (segment (start 209.866967 45.88441) (end 211.786967 43.96441) (width 0.4) (layer "F.Cu") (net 1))
 (segment (start 218.771967 44.91741) (end 217.818967 43.96441) (width 0.25) (layer "F.Cu") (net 1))
 (segment (start 218.241967 45.163567) (end 218.488124 44.91741) (width 0.25) (layer "B.Cu") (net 1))
 (segment (start 218.241967 46.96441) (end 218.241967 45.163567) (width 0.25) (layer "B.Cu") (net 1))
 (segment (start 218.488124 44.91741) (end 218.771967 44.91741) (width 0.25) (layer "B.Cu") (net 1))
 (segment (start 230.56 45.95) (end 230.05 45.44) (width 0.4) (layer "F.Cu") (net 4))
 (segment (start 230.071967 45.418033) (end 230.071967 40.866643) (width 0.4) (layer "F.Cu") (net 4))
 (segment (start 230.071967 40.866643) (end 229.365324 40.16) (width 0.4) (layer "F.Cu") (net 4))
 (segment (start 225.834466 40.16) (end 224.850876 39.17641) (width 0.4) (layer "F.Cu") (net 4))
 (segment (start 230.05 45.44) (end 230.071967 45.418033) (width 0.4) (layer "F.Cu") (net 4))
 (segment (start 229.365324 40.16) (end 225.834466 40.16) (width 0.4) (layer "F.Cu") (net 4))
 (via (at 230.56 45.95) (size 0.8) (drill 0.4) (layers "F.Cu" "B.Cu") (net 4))
 (segment (start 230.16059 46.34941) (end 230.56 45.95) (width 0.4) (layer "B.Cu") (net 4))
 (segment (start 229.541967 46.34941) (end 230.16059 46.34941) (width 0.4) (layer "B.Cu") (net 4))
 (segment (start 222.866967 46.188567) (end 221.59581 44.91741) (width 0.25) (layer "B.Cu") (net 2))
 (segment (start 218.241967 48.40441) (end 221.841967 48.40441) (width 0.25) (layer "B.Cu") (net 2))
 (segment (start 222.866967 48.32941) (end 222.866967 46.188567) (width 0.25) (layer "B.Cu") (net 2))
 (segment (start 221.59581 44.91741) (end 221.311967 44.91741) (width 0.25) (layer "B.Cu") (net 2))
 (segment (start 221.841967 48.40441) (end 222.791967 48.40441) (width 0.25) (layer "B.Cu") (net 2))
 (segment (start 222.791967 48.40441) (end 222.866967 48.32941) (width 0.25) (layer "B.Cu") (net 2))
 (segment (start 224.73059 49.32941) (end 225.86 48.2) (width 0.4) (layer "B.Cu") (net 3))
 (segment (start 209.736967 49.32941) (end 224.73059 49.32941) (width 0.4) (layer "B.Cu") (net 3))
 (segment (start 228.041967 47.49941) (end 228.041967 46.34941) (width 0.4) (layer "B.Cu") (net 3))
 (segment (start 225.86 48.2) (end 227.341377 48.2) (width 0.4) (layer "B.Cu") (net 3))
 (segment (start 208.291967 47.88441) (end 209.736967 49.32941) (width 0.4) (layer "B.Cu") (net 3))
 (segment (start 227.341377 48.2) (end 228.041967 47.49941) (width 0.4) (layer "B.Cu") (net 3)))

